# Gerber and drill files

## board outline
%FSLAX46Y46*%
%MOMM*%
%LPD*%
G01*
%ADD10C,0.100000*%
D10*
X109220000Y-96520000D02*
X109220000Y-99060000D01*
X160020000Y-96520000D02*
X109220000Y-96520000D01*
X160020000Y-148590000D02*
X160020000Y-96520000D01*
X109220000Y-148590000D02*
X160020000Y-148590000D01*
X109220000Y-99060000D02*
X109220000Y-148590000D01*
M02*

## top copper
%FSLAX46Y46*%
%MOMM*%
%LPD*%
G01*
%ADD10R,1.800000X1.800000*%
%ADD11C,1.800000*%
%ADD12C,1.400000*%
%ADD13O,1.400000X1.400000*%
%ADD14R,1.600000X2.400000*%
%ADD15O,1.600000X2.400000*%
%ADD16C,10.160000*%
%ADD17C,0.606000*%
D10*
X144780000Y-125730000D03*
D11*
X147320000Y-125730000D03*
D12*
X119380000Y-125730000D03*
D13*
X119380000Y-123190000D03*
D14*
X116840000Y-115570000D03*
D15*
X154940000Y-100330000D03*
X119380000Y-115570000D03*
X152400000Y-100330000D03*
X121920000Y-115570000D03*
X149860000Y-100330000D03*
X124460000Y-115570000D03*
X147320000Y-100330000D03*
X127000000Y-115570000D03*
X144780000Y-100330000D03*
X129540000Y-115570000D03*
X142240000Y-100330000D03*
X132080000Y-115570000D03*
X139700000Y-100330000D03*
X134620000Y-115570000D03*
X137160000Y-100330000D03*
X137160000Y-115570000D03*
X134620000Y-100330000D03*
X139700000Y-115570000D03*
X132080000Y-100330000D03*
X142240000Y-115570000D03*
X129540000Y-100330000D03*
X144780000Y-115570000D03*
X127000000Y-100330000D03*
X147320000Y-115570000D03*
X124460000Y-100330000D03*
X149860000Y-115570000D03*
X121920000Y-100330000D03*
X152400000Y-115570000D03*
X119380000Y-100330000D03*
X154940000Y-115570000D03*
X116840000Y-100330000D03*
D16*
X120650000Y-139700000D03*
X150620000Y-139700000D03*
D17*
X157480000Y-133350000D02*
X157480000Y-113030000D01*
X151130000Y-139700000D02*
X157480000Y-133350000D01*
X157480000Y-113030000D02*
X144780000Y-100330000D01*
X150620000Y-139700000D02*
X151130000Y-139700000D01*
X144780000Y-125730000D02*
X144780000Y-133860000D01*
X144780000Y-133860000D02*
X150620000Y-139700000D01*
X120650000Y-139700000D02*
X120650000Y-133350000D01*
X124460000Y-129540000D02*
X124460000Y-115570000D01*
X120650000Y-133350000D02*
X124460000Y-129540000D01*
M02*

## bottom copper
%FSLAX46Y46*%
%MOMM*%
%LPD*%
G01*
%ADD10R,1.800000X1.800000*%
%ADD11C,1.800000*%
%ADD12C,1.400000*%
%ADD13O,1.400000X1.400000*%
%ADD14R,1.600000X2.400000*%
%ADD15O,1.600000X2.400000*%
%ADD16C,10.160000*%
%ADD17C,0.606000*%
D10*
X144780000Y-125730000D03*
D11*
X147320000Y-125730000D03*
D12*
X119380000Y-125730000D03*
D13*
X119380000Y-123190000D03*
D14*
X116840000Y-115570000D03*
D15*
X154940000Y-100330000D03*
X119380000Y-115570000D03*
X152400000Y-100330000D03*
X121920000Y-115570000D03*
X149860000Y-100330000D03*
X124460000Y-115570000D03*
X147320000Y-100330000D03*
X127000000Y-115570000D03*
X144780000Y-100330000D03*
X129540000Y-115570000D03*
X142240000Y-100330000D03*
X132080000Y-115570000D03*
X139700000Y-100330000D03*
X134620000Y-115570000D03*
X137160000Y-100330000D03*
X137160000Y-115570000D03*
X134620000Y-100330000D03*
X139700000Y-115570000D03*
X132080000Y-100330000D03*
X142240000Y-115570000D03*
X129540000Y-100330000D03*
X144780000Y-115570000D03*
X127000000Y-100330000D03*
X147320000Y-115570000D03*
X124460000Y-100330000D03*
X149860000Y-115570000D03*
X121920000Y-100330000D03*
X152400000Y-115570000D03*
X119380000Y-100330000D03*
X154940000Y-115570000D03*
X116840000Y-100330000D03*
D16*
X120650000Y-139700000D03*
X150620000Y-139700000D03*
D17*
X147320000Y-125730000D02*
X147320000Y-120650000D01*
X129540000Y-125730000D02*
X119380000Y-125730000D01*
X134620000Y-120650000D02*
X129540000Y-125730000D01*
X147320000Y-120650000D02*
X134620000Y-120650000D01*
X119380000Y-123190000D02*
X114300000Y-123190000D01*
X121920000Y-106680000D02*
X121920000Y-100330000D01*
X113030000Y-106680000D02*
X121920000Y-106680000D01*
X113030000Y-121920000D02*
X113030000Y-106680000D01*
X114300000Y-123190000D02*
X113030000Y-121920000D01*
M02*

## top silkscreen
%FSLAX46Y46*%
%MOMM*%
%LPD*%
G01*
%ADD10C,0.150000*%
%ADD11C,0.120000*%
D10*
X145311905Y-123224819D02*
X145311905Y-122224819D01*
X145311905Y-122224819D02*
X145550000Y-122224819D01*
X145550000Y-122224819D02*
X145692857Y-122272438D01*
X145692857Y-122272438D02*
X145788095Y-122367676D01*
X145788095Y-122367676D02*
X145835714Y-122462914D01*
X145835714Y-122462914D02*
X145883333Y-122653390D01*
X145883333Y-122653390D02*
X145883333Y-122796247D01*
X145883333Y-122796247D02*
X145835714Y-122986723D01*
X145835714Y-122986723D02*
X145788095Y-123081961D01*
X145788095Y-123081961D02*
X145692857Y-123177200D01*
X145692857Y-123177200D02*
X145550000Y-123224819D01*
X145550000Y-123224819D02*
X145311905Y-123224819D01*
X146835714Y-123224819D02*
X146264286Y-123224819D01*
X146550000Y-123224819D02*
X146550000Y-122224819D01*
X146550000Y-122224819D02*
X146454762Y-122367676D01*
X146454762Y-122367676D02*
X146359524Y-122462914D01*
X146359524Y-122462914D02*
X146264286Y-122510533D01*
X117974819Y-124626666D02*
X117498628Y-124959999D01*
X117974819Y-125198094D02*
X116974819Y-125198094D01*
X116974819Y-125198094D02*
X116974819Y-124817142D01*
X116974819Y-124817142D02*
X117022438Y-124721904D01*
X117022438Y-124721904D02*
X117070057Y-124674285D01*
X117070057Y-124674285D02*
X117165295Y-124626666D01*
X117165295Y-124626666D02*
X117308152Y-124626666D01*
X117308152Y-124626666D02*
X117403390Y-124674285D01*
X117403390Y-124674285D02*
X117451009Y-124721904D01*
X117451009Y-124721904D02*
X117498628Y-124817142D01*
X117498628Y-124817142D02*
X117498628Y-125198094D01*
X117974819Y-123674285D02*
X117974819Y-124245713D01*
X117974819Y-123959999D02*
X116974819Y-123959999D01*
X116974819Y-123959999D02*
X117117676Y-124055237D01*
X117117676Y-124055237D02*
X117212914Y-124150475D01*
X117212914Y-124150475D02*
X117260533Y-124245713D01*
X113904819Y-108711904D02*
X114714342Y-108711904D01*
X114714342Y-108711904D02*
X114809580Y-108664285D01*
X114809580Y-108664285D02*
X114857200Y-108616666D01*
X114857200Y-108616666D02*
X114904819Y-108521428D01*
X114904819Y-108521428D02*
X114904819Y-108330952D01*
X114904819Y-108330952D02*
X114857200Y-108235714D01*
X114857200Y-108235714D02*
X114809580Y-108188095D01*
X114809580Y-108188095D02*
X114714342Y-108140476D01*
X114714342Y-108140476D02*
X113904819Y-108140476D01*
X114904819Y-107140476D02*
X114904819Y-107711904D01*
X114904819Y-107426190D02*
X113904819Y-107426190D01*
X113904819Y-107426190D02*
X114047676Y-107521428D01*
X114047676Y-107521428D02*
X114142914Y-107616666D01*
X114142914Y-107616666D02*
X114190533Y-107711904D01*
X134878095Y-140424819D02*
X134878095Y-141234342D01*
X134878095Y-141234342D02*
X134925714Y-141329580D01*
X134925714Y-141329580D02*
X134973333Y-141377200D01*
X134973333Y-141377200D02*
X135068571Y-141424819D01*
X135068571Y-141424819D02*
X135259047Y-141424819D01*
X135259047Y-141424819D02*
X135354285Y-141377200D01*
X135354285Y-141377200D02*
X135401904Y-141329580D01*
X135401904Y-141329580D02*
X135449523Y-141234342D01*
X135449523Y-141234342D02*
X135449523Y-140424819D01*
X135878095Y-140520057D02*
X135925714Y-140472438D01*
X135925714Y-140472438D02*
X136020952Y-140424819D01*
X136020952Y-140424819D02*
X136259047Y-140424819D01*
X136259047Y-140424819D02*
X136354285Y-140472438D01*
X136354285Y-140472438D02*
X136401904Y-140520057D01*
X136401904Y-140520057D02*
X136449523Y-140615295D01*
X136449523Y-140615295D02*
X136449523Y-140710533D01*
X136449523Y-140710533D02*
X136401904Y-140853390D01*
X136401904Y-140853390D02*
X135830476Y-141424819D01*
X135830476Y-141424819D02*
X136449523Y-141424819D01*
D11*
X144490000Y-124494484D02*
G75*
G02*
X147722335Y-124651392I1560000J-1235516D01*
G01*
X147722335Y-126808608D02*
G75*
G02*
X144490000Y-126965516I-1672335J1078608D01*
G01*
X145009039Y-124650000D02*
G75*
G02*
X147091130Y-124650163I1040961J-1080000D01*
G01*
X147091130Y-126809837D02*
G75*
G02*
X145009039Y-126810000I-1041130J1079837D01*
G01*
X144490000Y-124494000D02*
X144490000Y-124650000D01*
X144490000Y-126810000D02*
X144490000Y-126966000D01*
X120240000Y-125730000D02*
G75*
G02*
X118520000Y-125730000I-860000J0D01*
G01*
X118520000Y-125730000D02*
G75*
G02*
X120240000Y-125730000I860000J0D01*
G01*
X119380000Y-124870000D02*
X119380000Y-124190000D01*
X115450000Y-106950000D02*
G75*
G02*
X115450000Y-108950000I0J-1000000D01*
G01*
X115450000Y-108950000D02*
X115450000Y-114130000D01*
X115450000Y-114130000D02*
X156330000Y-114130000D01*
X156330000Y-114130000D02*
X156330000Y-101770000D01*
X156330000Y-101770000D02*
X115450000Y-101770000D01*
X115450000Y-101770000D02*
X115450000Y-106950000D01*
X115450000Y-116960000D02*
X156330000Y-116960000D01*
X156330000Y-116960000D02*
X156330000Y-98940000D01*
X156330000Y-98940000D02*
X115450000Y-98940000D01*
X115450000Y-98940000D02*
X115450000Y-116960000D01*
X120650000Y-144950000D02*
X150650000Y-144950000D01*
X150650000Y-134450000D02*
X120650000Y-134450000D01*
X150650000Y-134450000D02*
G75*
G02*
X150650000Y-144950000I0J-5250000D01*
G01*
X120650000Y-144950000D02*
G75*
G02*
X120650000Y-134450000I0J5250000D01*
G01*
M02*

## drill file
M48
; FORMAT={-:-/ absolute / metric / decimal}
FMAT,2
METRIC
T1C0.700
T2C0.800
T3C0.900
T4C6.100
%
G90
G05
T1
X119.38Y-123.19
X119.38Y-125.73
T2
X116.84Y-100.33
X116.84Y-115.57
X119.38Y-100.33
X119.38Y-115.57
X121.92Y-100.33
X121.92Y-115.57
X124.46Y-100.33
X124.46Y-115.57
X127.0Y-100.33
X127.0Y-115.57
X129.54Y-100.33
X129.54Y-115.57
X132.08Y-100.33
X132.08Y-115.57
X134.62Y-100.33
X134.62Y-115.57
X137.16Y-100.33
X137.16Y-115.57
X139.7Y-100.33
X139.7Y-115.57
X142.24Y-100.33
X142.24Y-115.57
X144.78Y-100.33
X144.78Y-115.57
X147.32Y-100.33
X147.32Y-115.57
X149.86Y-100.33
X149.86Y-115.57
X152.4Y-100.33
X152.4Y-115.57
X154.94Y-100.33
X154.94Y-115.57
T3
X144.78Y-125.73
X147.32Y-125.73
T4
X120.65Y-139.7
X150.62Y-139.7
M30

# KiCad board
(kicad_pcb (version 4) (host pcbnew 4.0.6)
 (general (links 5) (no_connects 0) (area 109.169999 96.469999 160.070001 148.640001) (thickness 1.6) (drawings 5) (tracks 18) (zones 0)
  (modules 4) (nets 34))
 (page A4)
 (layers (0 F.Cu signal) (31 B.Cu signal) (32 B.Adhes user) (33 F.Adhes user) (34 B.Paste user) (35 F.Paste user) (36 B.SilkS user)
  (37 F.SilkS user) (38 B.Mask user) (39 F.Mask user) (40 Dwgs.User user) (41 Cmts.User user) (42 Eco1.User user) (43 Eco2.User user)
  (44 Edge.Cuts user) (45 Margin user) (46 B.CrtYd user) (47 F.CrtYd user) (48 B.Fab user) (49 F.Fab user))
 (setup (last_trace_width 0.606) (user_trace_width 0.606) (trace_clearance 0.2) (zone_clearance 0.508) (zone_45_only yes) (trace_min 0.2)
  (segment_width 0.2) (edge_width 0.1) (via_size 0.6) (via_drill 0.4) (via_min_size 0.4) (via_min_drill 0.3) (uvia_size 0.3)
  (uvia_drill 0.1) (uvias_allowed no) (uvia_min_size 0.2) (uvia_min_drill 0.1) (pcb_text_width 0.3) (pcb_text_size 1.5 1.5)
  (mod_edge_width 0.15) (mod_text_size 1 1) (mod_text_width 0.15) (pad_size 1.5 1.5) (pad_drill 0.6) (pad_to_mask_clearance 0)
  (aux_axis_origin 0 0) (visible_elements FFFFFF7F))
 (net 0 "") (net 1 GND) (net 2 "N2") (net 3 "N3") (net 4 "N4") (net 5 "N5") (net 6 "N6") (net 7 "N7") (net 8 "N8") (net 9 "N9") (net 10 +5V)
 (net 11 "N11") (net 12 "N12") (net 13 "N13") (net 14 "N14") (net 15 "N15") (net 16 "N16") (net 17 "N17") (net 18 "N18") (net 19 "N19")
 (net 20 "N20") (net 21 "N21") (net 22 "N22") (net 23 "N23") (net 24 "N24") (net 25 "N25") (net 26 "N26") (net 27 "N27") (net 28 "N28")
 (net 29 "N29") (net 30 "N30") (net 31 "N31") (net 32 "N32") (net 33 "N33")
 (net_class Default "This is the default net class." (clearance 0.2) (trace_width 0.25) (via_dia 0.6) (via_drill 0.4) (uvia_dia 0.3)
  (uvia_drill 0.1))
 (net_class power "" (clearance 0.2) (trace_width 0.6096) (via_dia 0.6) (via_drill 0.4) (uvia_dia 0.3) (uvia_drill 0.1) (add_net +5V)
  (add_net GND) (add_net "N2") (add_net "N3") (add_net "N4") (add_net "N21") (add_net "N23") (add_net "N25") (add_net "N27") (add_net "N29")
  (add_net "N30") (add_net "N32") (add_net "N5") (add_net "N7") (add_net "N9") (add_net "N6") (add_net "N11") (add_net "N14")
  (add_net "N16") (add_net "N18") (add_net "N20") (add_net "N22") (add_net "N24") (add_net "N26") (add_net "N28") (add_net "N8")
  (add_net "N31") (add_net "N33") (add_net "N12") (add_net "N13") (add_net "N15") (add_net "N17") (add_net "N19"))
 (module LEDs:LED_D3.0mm (layer F.Cu) (at 144.78 125.73)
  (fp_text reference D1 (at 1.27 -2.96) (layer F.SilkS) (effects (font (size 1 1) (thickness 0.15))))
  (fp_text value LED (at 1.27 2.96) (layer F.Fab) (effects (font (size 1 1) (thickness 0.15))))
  (fp_arc (start 1.27 0) (end -0.29 -1.235516) (angle 108.8) (layer F.SilkS) (width 0.12))
  (fp_arc (start 1.27 0) (end -0.29 1.235516) (angle -108.8) (layer F.SilkS) (width 0.12))
  (fp_arc (start 1.27 0) (end 0.229039 -1.08) (angle 87.9) (layer F.SilkS) (width 0.12))
  (fp_arc (start 1.27 0) (end 0.229039 1.08) (angle -87.9) (layer F.SilkS) (width 0.12))
  (fp_line (start -0.29 -1.236) (end -0.29 -1.08) (layer F.SilkS) (width 0.12))
  (fp_line (start -0.29 1.08) (end -0.29 1.236) (layer F.SilkS) (width 0.12))
  (pad 1 thru_hole rect (at 0 0) (size 1.8 1.8) (drill 0.9) (layers *.Cu *.Mask) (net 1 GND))
  (pad 2 thru_hole circle (at 2.54 0) (size 1.8 1.8) (drill 0.9) (layers *.Cu *.Mask) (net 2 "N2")))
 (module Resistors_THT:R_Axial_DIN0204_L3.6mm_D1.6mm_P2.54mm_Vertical (layer F.Cu) (at 119.38 125.73 90)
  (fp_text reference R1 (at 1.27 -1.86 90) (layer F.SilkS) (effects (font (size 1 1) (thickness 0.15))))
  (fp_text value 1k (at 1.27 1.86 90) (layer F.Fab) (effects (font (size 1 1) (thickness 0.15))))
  (fp_circle (center 0 0) (end 0.86 0) (layer F.SilkS) (width 0.12))
  (fp_line (start 0.86 0) (end 1.54 0) (layer F.SilkS) (width 0.12))
  (pad 1 thru_hole circle (at 0 0 90) (size 1.4 1.4) (drill 0.7) (layers *.Cu *.Mask) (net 2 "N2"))
  (pad 2 thru_hole oval (at 2.54 0 90) (size 1.4 1.4) (drill 0.7) (layers *.Cu *.Mask) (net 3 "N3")))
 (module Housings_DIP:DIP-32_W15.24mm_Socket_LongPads (layer F.Cu) (at 116.84 115.57 90)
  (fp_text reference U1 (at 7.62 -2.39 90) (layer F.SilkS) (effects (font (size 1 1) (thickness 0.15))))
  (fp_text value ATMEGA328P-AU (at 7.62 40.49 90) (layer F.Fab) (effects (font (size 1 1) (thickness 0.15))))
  (fp_arc (start 7.62 -1.39) (end 6.62 -1.39) (angle -180) (layer F.SilkS) (width 0.12))
  (fp_line (start 6.62 -1.39) (end 1.44 -1.39) (layer F.SilkS) (width 0.12))
  (fp_line (start 1.44 -1.39) (end 1.44 39.49) (layer F.SilkS) (width 0.12))
  (fp_line (start 1.44 39.49) (end 13.8 39.49) (layer F.SilkS) (width 0.12))
  (fp_line (start 13.8 39.49) (end 13.8 -1.39) (layer F.SilkS) (width 0.12))
  (fp_line (start 13.8 -1.39) (end 8.62 -1.39) (layer F.SilkS) (width 0.12))
  (fp_line (start -1.39 -1.39) (end -1.39 39.49) (layer F.SilkS) (width 0.12))
  (fp_line (start -1.39 39.49) (end 16.63 39.49) (layer F.SilkS) (width 0.12))
  (fp_line (start 16.63 39.49) (end 16.63 -1.39) (layer F.SilkS) (width 0.12))
  (fp_line (start 16.63 -1.39) (end -1.39 -1.39) (layer F.SilkS) (width 0.12))
  (pad 1 thru_hole rect (at 0 0 90) (size 2.4 1.6) (drill 0.8) (layers *.Cu *.Mask) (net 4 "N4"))
  (pad 17 thru_hole oval (at 15.24 38.1 90) (size 2.4 1.6) (drill 0.8) (layers *.Cu *.Mask) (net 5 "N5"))
  (pad 2 thru_hole oval (at 0 2.54 90) (size 2.4 1.6) (drill 0.8) (layers *.Cu *.Mask) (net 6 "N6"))
  (pad 18 thru_hole oval (at 15.24 35.56 90) (size 2.4 1.6) (drill 0.8) (layers *.Cu *.Mask) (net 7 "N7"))
  (pad 3 thru_hole oval (at 0 5.08 90) (size 2.4 1.6) (drill 0.8) (layers *.Cu *.Mask) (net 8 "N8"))
  (pad 19 thru_hole oval (at 15.24 33.02 90) (size 2.4 1.6) (drill 0.8) (layers *.Cu *.Mask) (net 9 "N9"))
  (pad 4 thru_hole oval (at 0 7.62 90) (size 2.4 1.6) (drill 0.8) (layers *.Cu *.Mask) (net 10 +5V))
  (pad 20 thru_hole oval (at 15.24 30.48 90) (size 2.4 1.6) (drill 0.8) (layers *.Cu *.Mask) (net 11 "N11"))
  (pad 5 thru_hole oval (at 0 10.16 90) (size 2.4 1.6) (drill 0.8) (layers *.Cu *.Mask) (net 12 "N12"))
  (pad 21 thru_hole oval (at 15.24 27.94 90) (size 2.4 1.6) (drill 0.8) (layers *.Cu *.Mask) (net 1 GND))
  (pad 6 thru_hole oval (at 0 12.7 90) (size 2.4 1.6) (drill 0.8) (layers *.Cu *.Mask) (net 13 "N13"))
  (pad 22 thru_hole oval (at 15.24 25.4 90) (size 2.4 1.6) (drill 0.8) (layers *.Cu *.Mask) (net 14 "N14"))
  (pad 7 thru_hole oval (at 0 15.24 90) (size 2.4 1.6) (drill 0.8) (layers *.Cu *.Mask) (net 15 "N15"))
  (pad 23 thru_hole oval (at 15.24 22.86 90) (size 2.4 1.6) (drill 0.8) (layers *.Cu *.Mask) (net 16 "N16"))
  (pad 8 thru_hole oval (at 0 17.78 90) (size 2.4 1.6) (drill 0.8) (layers *.Cu *.Mask) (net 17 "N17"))
  (pad 24 thru_hole oval (at 15.24 20.32 90) (size 2.4 1.6) (drill 0.8) (layers *.Cu *.Mask) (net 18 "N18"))
  (pad 9 thru_hole oval (at 0 20.32 90) (size 2.4 1.6) (drill 0.8) (layers *.Cu *.Mask) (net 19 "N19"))
  (pad 25 thru_hole oval (at 15.24 17.78 90) (size 2.4 1.6) (drill 0.8) (layers *.Cu *.Mask) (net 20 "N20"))
  (pad 10 thru_hole oval (at 0 22.86 90) (size 2.4 1.6) (drill 0.8) (layers *.Cu *.Mask) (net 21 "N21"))
  (pad 26 thru_hole oval (at 15.24 15.24 90) (size 2.4 1.6) (drill 0.8) (layers *.Cu *.Mask) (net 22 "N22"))
  (pad 11 thru_hole oval (at 0 25.4 90) (size 2.4 1.6) (drill 0.8) (layers *.Cu *.Mask) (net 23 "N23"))
  (pad 27 thru_hole oval (at 15.24 12.7 90) (size 2.4 1.6) (drill 0.8) (layers *.Cu *.Mask) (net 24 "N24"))
  (pad 12 thru_hole oval (at 0 27.94 90) (size 2.4 1.6) (drill 0.8) (layers *.Cu *.Mask) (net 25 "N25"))
  (pad 28 thru_hole oval (at 15.24 10.16 90) (size 2.4 1.6) (drill 0.8) (layers *.Cu *.Mask) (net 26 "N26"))
  (pad 13 thru_hole oval (at 0 30.48 90) (size 2.4 1.6) (drill 0.8) (layers *.Cu *.Mask) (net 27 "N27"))
  (pad 29 thru_hole oval (at 15.24 7.62 90) (size 2.4 1.6) (drill 0.8) (layers *.Cu *.Mask) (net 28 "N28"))
  (pad 14 thru_hole oval (at 0 33.02 90) (size 2.4 1.6) (drill 0.8) (layers *.Cu *.Mask) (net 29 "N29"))
  (pad 30 thru_hole oval (at 15.24 5.08 90) (size 2.4 1.6) (drill 0.8) (layers *.Cu *.Mask) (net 3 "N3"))
  (pad 15 thru_hole oval (at 0 35.56 90) (size 2.4 1.6) (drill 0.8) (layers *.Cu *.Mask) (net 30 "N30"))
  (pad 31 thru_hole oval (at 15.24 2.54 90) (size 2.4 1.6) (drill 0.8) (layers *.Cu *.Mask) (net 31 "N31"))
  (pad 16 thru_hole oval (at 0 38.1 90) (size 2.4 1.6) (drill 0.8) (layers *.Cu *.Mask) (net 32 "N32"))
  (pad 32 thru_hole oval (at 15.24 0 90) (size 2.4 1.6) (drill 0.8) (layers *.Cu *.Mask) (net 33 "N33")))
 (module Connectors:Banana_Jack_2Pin (layer F.Cu) (at 120.65 139.7)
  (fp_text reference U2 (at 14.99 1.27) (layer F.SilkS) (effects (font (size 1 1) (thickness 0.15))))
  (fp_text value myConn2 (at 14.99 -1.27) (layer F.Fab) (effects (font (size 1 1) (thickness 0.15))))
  (fp_line (start 0 5.25) (end 30 5.25) (layer F.SilkS) (width 0.12))
  (fp_line (start 30 -5.25) (end 0 -5.25) (layer F.SilkS) (width 0.12))
  (fp_arc (start 30 0) (end 30 -5.25) (angle 180) (layer F.SilkS) (width 0.12))
  (fp_arc (start 0 0) (end 0 5.25) (angle 180) (layer F.SilkS) (width 0.12))
  (pad 1 thru_hole circle (at 0 0) (size 10.16 10.16) (drill 6.1) (layers *.Cu *.Mask) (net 10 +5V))
  (pad 2 thru_hole circle (at 29.97 0) (size 10.16 10.16) (drill 6.1) (layers *.Cu *.Mask) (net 1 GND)))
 (gr_line (start 109.22 96.52) (end 109.22 99.06) (angle 90) (layer Edge.Cuts) (width 0.1))
 (gr_line (start 160.02 96.52) (end 109.22 96.52) (angle 90) (layer Edge.Cuts) (width 0.1))
 (gr_line (start 160.02 148.59) (end 160.02 96.52) (angle 90) (layer Edge.Cuts) (width 0.1))
 (gr_line (start 109.22 148.59) (end 160.02 148.59) (angle 90) (layer Edge.Cuts) (width 0.1))
 (gr_line (start 109.22 99.06) (end 109.22 148.59) (angle 90) (layer Edge.Cuts) (width 0.1))
 (segment (start 157.48 133.35) (end 157.48 113.03) (width 0.606) (layer F.Cu) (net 1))
 (segment (start 151.13 139.7) (end 157.48 133.35) (width 0.606) (layer F.Cu) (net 1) (status 400000))
 (segment (start 157.48 113.03) (end 144.78 100.33) (width 0.606) (layer F.Cu) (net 1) (status 800000))
 (segment (start 150.62 139.7) (end 151.13 139.7) (width 0.606) (layer F.Cu) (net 1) (status C00000))
 (segment (start 144.78 125.73) (end 144.78 133.86) (width 0.606) (layer F.Cu) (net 1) (status 400000))
 (segment (start 144.78 133.86) (end 150.62 139.7) (width 0.606) (layer F.Cu) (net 1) (status 800000))
 (segment (start 147.32 125.73) (end 147.32 120.65) (width 0.606) (layer B.Cu) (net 2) (status 400000))
 (segment (start 129.54 125.73) (end 119.38 125.73) (width 0.606) (layer B.Cu) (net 2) (status 800000))
 (segment (start 134.62 120.65) (end 129.54 125.73) (width 0.606) (layer B.Cu) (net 2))
 (segment (start 147.32 120.65) (end 134.62 120.65) (width 0.606) (layer B.Cu) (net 2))
 (segment (start 119.38 123.19) (end 114.3 123.19) (width 0.606) (layer B.Cu) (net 3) (status 400000))
 (segment (start 121.92 106.68) (end 121.92 100.33) (width 0.606) (layer B.Cu) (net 3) (status 800000))
 (segment (start 113.03 106.68) (end 121.92 106.68) (width 0.606) (layer B.Cu) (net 3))
 (segment (start 113.03 121.92) (end 113.03 106.68) (width 0.606) (layer B.Cu) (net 3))
 (segment (start 114.3 123.19) (end 113.03 121.92) (width 0.606) (layer B.Cu) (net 3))
 (segment (start 120.65 139.7) (end 120.65 133.35) (width 0.606) (layer F.Cu) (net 10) (status 400000))
 (segment (start 124.46 129.54) (end 124.46 115.57) (width 0.606) (layer F.Cu) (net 10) (status 800000))
 (segment (start 120.65 133.35) (end 124.46 129.54) (width 0.606) (layer F.Cu) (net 10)))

